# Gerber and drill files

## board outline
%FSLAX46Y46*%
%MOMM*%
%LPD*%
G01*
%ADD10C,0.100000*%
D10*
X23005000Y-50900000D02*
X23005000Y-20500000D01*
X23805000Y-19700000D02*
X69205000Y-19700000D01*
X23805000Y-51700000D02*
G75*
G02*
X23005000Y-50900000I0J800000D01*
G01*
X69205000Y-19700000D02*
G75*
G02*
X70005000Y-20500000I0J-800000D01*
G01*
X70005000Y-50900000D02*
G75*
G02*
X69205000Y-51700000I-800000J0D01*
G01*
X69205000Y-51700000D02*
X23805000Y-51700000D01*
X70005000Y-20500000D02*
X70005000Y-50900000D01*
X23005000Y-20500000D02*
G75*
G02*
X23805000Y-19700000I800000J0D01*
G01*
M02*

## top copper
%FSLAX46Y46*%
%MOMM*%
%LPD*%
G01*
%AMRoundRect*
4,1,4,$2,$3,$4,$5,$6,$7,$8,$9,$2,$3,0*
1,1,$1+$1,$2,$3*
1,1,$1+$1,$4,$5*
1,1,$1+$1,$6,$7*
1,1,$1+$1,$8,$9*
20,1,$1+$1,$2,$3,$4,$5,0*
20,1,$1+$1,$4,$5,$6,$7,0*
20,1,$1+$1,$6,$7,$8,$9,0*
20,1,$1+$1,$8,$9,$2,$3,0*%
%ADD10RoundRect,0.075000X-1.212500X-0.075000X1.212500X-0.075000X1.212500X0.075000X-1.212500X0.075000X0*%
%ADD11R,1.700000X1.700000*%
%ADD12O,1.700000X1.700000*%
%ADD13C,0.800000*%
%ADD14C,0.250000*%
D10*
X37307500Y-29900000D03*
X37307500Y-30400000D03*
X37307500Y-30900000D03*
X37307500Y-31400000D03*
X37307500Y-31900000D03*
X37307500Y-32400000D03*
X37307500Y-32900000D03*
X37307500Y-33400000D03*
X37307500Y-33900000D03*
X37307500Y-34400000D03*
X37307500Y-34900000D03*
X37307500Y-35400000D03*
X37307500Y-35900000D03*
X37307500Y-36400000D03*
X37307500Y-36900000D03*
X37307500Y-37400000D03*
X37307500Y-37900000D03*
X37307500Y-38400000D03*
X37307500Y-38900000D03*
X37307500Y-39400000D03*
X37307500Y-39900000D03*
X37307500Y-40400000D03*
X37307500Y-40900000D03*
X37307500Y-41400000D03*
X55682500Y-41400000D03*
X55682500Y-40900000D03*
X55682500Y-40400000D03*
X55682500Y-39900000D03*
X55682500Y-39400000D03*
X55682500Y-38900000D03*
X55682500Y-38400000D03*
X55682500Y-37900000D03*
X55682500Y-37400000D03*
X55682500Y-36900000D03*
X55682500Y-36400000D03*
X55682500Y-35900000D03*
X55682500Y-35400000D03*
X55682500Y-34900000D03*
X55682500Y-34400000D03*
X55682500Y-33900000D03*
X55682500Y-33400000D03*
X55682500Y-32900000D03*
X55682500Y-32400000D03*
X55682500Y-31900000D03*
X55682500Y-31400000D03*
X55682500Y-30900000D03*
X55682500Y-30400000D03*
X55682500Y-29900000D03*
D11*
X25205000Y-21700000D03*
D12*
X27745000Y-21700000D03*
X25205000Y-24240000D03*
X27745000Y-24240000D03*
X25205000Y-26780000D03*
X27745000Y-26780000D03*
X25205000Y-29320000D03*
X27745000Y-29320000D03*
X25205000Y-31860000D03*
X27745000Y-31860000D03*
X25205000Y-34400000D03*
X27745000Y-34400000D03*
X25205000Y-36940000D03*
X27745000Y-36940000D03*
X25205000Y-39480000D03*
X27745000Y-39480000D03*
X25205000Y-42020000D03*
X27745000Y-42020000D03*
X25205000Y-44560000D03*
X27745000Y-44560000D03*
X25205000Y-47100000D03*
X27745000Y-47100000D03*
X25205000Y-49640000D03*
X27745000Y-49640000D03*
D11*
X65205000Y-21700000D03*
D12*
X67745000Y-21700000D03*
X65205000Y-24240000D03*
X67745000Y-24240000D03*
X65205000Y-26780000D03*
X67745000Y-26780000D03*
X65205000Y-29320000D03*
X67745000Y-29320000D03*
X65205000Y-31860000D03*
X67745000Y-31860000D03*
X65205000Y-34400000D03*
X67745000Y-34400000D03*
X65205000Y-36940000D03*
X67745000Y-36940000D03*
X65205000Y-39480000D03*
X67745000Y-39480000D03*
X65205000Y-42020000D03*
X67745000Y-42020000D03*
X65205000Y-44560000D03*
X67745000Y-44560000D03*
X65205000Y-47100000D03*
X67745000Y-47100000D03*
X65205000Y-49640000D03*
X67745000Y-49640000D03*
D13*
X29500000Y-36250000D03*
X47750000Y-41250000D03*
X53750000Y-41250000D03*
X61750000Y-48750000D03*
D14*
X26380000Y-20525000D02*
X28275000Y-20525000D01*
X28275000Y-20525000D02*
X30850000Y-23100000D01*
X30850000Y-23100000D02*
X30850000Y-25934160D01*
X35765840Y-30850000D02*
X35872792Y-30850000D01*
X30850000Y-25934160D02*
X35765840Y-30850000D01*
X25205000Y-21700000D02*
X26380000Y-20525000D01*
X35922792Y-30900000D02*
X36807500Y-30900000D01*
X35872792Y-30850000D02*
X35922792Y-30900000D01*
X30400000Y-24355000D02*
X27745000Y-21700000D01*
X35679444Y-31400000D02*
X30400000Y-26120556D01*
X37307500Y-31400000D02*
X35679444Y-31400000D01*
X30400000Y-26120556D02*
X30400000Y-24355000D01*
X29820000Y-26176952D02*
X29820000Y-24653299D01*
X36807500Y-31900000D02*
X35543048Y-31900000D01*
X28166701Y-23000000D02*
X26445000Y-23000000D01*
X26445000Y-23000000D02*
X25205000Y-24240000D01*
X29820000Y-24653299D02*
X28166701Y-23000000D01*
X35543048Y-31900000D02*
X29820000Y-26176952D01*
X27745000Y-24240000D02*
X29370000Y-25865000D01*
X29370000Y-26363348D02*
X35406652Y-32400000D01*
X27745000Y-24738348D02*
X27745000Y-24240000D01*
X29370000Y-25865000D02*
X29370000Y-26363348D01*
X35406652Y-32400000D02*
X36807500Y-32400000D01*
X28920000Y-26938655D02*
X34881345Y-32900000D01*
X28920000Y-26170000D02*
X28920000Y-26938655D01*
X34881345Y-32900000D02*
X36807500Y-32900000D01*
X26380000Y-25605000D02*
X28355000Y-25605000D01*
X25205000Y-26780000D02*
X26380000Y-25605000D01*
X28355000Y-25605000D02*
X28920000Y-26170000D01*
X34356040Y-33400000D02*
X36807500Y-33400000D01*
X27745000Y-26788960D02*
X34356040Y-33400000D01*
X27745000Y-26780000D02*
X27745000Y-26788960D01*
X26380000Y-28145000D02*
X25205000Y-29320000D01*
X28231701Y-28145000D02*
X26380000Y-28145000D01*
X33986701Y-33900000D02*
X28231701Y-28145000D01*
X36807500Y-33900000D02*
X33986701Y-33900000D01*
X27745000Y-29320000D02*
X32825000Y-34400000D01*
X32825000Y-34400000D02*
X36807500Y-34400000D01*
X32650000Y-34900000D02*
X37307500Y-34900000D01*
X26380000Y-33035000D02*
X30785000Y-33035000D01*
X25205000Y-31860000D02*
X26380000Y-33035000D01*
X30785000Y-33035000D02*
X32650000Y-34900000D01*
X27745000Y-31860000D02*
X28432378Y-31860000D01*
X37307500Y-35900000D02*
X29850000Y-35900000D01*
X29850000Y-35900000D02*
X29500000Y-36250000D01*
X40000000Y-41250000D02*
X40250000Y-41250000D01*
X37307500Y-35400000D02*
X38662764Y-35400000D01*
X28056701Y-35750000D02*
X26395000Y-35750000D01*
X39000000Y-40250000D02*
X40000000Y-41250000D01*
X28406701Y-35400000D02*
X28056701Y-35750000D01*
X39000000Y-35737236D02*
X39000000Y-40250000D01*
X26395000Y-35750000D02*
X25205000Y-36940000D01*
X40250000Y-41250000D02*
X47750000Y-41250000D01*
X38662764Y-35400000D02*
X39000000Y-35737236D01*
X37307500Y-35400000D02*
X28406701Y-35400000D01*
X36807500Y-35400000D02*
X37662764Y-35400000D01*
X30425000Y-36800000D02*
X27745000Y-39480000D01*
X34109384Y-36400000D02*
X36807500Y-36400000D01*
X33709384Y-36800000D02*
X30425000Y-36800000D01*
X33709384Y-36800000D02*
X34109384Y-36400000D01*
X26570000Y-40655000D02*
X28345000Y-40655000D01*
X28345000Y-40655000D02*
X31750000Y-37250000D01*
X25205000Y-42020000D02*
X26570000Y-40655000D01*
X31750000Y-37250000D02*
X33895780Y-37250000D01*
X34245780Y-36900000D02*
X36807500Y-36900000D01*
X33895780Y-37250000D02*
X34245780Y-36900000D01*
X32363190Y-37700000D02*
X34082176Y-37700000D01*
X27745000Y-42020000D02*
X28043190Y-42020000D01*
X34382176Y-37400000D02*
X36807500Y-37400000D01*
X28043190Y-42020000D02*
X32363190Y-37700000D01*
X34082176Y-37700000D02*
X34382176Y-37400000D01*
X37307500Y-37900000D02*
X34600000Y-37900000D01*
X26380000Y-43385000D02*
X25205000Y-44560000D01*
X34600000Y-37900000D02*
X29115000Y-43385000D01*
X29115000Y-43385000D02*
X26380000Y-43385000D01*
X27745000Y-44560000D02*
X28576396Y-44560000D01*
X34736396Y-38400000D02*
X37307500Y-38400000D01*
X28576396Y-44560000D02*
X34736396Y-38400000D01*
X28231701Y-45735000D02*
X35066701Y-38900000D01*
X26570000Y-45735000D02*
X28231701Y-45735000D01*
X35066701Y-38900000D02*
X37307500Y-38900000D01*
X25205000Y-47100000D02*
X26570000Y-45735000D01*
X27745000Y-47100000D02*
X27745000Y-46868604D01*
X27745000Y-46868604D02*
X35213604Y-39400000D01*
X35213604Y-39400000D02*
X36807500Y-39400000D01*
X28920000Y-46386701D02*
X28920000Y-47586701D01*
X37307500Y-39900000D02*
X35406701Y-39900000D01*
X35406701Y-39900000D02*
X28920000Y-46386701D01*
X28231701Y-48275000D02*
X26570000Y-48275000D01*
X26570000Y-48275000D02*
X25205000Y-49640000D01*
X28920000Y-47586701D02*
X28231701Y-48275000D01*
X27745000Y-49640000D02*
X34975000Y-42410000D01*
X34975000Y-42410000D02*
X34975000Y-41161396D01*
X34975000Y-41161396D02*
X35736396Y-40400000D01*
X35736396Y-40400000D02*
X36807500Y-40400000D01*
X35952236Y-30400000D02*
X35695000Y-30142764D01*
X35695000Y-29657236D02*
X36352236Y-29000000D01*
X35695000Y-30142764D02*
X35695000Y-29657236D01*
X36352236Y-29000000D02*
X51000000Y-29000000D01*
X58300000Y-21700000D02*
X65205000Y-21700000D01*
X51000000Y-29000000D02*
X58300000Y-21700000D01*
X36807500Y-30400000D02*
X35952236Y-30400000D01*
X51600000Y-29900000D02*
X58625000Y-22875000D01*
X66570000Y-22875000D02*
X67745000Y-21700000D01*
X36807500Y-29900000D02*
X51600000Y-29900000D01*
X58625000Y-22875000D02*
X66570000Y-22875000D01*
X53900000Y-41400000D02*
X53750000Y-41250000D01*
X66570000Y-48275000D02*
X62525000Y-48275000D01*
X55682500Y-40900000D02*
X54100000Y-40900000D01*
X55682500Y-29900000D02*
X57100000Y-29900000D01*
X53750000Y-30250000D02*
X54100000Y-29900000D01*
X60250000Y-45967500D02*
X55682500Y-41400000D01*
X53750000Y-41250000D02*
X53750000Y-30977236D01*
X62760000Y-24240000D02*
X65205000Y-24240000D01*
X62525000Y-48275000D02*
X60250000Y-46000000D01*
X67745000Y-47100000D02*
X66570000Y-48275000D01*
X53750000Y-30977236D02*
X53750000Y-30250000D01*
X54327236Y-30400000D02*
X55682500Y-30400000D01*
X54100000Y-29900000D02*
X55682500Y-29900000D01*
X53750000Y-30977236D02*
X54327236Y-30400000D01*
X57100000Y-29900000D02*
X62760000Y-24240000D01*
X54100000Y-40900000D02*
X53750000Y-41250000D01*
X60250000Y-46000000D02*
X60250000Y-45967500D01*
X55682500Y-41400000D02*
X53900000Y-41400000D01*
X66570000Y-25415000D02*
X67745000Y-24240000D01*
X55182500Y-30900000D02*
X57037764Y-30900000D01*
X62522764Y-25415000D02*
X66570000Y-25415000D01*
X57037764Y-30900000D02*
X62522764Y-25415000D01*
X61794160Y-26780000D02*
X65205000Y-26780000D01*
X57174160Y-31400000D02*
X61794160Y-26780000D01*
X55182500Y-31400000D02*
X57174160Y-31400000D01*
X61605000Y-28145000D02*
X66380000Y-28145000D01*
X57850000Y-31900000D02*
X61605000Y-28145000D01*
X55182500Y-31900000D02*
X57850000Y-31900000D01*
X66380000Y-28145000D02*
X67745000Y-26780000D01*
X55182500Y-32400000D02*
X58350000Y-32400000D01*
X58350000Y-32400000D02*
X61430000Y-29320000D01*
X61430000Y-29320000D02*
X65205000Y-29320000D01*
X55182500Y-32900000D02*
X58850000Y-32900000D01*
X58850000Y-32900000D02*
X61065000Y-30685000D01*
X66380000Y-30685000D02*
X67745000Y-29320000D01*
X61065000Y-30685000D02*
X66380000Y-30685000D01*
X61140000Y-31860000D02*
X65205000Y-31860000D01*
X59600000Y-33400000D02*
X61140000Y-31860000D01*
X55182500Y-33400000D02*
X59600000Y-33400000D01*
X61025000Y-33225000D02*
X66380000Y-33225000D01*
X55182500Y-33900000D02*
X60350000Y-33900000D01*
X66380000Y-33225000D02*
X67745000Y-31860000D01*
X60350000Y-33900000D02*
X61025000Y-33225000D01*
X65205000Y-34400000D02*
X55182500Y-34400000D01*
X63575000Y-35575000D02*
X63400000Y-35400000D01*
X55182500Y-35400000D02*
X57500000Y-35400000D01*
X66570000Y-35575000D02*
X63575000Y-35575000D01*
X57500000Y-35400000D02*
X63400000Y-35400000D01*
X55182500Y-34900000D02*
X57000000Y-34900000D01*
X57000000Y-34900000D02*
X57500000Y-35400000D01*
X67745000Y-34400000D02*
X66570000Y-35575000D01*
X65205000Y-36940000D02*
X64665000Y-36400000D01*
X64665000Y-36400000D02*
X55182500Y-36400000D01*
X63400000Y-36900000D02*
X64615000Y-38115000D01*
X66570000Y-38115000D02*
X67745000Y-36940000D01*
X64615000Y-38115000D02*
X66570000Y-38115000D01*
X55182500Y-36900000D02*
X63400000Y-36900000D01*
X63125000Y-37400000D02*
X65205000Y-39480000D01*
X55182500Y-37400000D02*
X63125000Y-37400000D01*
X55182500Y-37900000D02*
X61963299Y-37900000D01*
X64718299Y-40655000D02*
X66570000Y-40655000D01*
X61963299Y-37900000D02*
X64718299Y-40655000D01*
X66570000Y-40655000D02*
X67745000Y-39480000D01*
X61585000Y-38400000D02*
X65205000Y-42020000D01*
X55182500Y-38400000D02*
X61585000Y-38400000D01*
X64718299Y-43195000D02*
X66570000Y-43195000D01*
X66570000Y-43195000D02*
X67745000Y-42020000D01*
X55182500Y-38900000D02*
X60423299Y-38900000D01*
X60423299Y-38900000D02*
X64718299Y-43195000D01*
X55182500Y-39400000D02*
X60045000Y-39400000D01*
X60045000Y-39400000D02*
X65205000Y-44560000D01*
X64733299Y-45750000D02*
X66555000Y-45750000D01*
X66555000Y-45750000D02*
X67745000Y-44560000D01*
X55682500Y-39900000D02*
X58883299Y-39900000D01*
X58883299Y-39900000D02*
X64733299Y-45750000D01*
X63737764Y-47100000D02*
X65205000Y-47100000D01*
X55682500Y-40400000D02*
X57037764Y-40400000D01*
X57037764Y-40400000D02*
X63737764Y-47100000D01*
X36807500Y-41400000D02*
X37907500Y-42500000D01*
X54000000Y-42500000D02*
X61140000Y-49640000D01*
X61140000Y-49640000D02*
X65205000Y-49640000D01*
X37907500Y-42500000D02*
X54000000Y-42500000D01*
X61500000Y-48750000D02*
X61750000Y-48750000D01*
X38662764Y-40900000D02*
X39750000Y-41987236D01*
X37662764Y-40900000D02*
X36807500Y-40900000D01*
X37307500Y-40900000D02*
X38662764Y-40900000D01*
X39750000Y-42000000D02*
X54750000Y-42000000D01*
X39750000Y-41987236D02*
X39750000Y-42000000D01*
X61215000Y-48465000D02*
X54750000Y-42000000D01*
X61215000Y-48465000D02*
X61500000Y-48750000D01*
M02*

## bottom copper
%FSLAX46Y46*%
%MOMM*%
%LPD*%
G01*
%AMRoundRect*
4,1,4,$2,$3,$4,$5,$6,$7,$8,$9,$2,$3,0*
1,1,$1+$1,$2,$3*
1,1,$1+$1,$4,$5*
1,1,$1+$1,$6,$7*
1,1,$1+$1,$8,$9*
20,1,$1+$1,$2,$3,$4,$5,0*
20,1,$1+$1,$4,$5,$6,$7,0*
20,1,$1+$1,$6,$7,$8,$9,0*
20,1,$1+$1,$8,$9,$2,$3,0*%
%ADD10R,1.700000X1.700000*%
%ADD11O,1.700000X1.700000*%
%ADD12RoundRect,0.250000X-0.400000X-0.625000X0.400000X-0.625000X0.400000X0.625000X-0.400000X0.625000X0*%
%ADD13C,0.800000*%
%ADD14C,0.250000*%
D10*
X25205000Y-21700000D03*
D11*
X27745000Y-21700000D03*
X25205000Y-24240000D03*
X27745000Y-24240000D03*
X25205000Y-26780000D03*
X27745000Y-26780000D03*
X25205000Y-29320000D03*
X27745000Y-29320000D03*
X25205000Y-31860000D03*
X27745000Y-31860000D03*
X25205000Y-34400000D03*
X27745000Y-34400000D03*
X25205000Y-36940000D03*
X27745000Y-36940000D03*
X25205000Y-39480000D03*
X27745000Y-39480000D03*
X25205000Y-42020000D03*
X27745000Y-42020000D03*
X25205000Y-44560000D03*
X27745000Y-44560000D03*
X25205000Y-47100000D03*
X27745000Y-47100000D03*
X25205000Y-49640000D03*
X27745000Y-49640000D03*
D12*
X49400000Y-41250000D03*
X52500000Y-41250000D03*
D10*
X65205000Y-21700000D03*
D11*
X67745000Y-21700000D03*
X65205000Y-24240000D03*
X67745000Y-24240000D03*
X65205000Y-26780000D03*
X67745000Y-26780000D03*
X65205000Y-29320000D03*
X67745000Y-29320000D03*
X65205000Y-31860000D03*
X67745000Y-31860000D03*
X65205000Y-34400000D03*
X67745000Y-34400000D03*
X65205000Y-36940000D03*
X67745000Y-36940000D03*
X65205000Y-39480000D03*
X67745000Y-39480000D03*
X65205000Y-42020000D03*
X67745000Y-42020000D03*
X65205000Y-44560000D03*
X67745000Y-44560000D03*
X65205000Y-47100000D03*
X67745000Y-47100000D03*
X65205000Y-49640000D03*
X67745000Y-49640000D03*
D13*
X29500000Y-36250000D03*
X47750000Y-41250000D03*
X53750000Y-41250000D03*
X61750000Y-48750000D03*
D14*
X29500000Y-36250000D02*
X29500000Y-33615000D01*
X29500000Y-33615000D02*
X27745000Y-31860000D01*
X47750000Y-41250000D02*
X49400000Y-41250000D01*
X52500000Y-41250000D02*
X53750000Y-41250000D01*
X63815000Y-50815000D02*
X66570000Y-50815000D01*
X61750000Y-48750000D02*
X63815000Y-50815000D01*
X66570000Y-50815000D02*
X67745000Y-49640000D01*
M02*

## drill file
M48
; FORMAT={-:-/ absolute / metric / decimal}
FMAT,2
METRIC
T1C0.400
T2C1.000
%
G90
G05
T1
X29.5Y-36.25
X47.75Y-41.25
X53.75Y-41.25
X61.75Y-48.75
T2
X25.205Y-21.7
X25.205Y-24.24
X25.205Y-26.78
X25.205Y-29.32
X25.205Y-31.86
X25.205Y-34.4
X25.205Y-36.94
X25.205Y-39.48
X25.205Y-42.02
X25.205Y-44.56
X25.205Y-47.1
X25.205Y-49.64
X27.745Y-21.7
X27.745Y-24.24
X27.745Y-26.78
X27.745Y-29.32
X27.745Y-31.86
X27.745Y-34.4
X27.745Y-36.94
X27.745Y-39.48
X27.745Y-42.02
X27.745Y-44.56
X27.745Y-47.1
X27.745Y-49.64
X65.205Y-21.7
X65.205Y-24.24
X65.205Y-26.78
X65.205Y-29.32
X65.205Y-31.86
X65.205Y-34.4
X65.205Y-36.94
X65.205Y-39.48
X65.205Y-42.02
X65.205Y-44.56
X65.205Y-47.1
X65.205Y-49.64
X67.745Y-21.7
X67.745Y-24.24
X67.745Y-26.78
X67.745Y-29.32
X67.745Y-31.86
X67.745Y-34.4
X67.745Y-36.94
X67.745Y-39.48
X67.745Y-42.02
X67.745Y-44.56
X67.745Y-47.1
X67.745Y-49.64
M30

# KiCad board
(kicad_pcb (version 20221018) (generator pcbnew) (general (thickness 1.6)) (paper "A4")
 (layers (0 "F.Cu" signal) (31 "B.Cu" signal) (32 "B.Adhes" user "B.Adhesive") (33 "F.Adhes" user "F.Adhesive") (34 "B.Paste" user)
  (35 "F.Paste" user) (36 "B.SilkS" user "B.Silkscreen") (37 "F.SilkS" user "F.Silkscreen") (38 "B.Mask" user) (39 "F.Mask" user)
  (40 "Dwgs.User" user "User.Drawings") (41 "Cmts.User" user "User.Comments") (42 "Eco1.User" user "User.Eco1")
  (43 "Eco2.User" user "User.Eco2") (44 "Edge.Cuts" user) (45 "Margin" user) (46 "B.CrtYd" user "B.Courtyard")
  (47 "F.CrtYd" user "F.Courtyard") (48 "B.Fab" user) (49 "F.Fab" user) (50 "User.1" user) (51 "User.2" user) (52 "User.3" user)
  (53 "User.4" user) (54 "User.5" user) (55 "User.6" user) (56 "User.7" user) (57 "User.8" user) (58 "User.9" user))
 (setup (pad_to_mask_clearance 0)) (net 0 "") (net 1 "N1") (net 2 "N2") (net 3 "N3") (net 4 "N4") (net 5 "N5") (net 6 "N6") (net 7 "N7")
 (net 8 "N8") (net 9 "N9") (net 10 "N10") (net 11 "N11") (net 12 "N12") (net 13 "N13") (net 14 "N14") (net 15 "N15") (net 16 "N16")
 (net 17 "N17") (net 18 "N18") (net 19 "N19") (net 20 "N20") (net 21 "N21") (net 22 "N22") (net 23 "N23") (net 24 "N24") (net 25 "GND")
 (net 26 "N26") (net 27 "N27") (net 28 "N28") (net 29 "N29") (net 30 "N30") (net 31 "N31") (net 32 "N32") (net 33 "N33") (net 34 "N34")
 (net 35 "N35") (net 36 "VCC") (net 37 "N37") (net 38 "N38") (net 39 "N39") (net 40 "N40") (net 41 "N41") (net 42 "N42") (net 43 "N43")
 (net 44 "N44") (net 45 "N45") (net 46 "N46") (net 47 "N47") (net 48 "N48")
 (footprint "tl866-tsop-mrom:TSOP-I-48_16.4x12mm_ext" (layer "F.Cu") (at 46.495 35.65)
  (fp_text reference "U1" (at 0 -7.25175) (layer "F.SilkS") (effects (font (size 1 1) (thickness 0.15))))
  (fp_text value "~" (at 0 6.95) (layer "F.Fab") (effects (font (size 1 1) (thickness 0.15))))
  (pad "1" smd roundrect (at -9.1875 -5.75) (size 2.575 0.3) (layers "F.Cu" "F.Paste" "F.Mask") (roundrect_rratio 0.25) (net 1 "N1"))
  (pad "2" smd roundrect (at -9.1875 -5.25) (size 2.575 0.3) (layers "F.Cu" "F.Paste" "F.Mask") (roundrect_rratio 0.25) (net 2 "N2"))
  (pad "3" smd roundrect (at -9.1875 -4.75) (size 2.575 0.3) (layers "F.Cu" "F.Paste" "F.Mask") (roundrect_rratio 0.25) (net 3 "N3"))
  (pad "4" smd roundrect (at -9.1875 -4.25) (size 2.575 0.3) (layers "F.Cu" "F.Paste" "F.Mask") (roundrect_rratio 0.25) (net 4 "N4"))
  (pad "5" smd roundrect (at -9.1875 -3.75) (size 2.575 0.3) (layers "F.Cu" "F.Paste" "F.Mask") (roundrect_rratio 0.25) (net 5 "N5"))
  (pad "6" smd roundrect (at -9.1875 -3.25) (size 2.575 0.3) (layers "F.Cu" "F.Paste" "F.Mask") (roundrect_rratio 0.25) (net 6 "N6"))
  (pad "7" smd roundrect (at -9.1875 -2.75) (size 2.575 0.3) (layers "F.Cu" "F.Paste" "F.Mask") (roundrect_rratio 0.25) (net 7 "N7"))
  (pad "8" smd roundrect (at -9.1875 -2.25) (size 2.575 0.3) (layers "F.Cu" "F.Paste" "F.Mask") (roundrect_rratio 0.25) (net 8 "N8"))
  (pad "9" smd roundrect (at -9.1875 -1.75) (size 2.575 0.3) (layers "F.Cu" "F.Paste" "F.Mask") (roundrect_rratio 0.25) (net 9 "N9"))
  (pad "10" smd roundrect (at -9.1875 -1.25) (size 2.575 0.3) (layers "F.Cu" "F.Paste" "F.Mask") (roundrect_rratio 0.25) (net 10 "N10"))
  (pad "11" smd roundrect (at -9.1875 -0.75) (size 2.575 0.3) (layers "F.Cu" "F.Paste" "F.Mask") (roundrect_rratio 0.25) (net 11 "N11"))
  (pad "12" smd roundrect (at -9.1875 -0.25) (size 2.575 0.3) (layers "F.Cu" "F.Paste" "F.Mask") (roundrect_rratio 0.25) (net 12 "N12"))
  (pad "13" smd roundrect (at -9.1875 0.25) (size 2.575 0.3) (layers "F.Cu" "F.Paste" "F.Mask") (roundrect_rratio 0.25) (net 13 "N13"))
  (pad "14" smd roundrect (at -9.1875 0.75) (size 2.575 0.3) (layers "F.Cu" "F.Paste" "F.Mask") (roundrect_rratio 0.25) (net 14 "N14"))
  (pad "15" smd roundrect (at -9.1875 1.25) (size 2.575 0.3) (layers "F.Cu" "F.Paste" "F.Mask") (roundrect_rratio 0.25) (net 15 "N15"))
  (pad "16" smd roundrect (at -9.1875 1.75) (size 2.575 0.3) (layers "F.Cu" "F.Paste" "F.Mask") (roundrect_rratio 0.25) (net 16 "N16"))
  (pad "17" smd roundrect (at -9.1875 2.25) (size 2.575 0.3) (layers "F.Cu" "F.Paste" "F.Mask") (roundrect_rratio 0.25) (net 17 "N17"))
  (pad "18" smd roundrect (at -9.1875 2.75) (size 2.575 0.3) (layers "F.Cu" "F.Paste" "F.Mask") (roundrect_rratio 0.25) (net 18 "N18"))
  (pad "19" smd roundrect (at -9.1875 3.25) (size 2.575 0.3) (layers "F.Cu" "F.Paste" "F.Mask") (roundrect_rratio 0.25) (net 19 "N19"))
  (pad "20" smd roundrect (at -9.1875 3.75) (size 2.575 0.3) (layers "F.Cu" "F.Paste" "F.Mask") (roundrect_rratio 0.25) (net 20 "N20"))
  (pad "21" smd roundrect (at -9.1875 4.25) (size 2.575 0.3) (layers "F.Cu" "F.Paste" "F.Mask") (roundrect_rratio 0.25) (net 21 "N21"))
  (pad "22" smd roundrect (at -9.1875 4.75) (size 2.575 0.3) (layers "F.Cu" "F.Paste" "F.Mask") (roundrect_rratio 0.25) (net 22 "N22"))
  (pad "23" smd roundrect (at -9.1875 5.25) (size 2.575 0.3) (layers "F.Cu" "F.Paste" "F.Mask") (roundrect_rratio 0.25) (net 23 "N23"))
  (pad "24" smd roundrect (at -9.1875 5.75) (size 2.575 0.3) (layers "F.Cu" "F.Paste" "F.Mask") (roundrect_rratio 0.25) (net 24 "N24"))
  (pad "25" smd roundrect (at 9.1875 5.75) (size 2.575 0.3) (layers "F.Cu" "F.Paste" "F.Mask") (roundrect_rratio 0.25) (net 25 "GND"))
  (pad "26" smd roundrect (at 9.1875 5.25) (size 2.575 0.3) (layers "F.Cu" "F.Paste" "F.Mask") (roundrect_rratio 0.25) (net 25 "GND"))
  (pad "27" smd roundrect (at 9.1875 4.75) (size 2.575 0.3) (layers "F.Cu" "F.Paste" "F.Mask") (roundrect_rratio 0.25) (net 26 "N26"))
  (pad "28" smd roundrect (at 9.1875 4.25) (size 2.575 0.3) (layers "F.Cu" "F.Paste" "F.Mask") (roundrect_rratio 0.25) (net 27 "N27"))
  (pad "29" smd roundrect (at 9.1875 3.75) (size 2.575 0.3) (layers "F.Cu" "F.Paste" "F.Mask") (roundrect_rratio 0.25) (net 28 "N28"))
  (pad "30" smd roundrect (at 9.1875 3.25) (size 2.575 0.3) (layers "F.Cu" "F.Paste" "F.Mask") (roundrect_rratio 0.25) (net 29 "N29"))
  (pad "31" smd roundrect (at 9.1875 2.75) (size 2.575 0.3) (layers "F.Cu" "F.Paste" "F.Mask") (roundrect_rratio 0.25) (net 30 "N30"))
  (pad "32" smd roundrect (at 9.1875 2.25) (size 2.575 0.3) (layers "F.Cu" "F.Paste" "F.Mask") (roundrect_rratio 0.25) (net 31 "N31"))
  (pad "33" smd roundrect (at 9.1875 1.75) (size 2.575 0.3) (layers "F.Cu" "F.Paste" "F.Mask") (roundrect_rratio 0.25) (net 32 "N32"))
  (pad "34" smd roundrect (at 9.1875 1.25) (size 2.575 0.3) (layers "F.Cu" "F.Paste" "F.Mask") (roundrect_rratio 0.25) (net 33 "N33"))
  (pad "35" smd roundrect (at 9.1875 0.75) (size 2.575 0.3) (layers "F.Cu" "F.Paste" "F.Mask") (roundrect_rratio 0.25) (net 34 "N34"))
  (pad "36" smd roundrect (at 9.1875 0.25) (size 2.575 0.3) (layers "F.Cu" "F.Paste" "F.Mask") (roundrect_rratio 0.25) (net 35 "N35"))
  (pad "37" smd roundrect (at 9.1875 -0.25) (size 2.575 0.3) (layers "F.Cu" "F.Paste" "F.Mask") (roundrect_rratio 0.25) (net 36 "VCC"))
  (pad "38" smd roundrect (at 9.1875 -0.75) (size 2.575 0.3) (layers "F.Cu" "F.Paste" "F.Mask") (roundrect_rratio 0.25) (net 36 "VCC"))
  (pad "39" smd roundrect (at 9.1875 -1.25) (size 2.575 0.3) (layers "F.Cu" "F.Paste" "F.Mask") (roundrect_rratio 0.25) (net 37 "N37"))
  (pad "40" smd roundrect (at 9.1875 -1.75) (size 2.575 0.3) (layers "F.Cu" "F.Paste" "F.Mask") (roundrect_rratio 0.25) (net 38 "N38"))
  (pad "41" smd roundrect (at 9.1875 -2.25) (size 2.575 0.3) (layers "F.Cu" "F.Paste" "F.Mask") (roundrect_rratio 0.25) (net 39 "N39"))
  (pad "42" smd roundrect (at 9.1875 -2.75) (size 2.575 0.3) (layers "F.Cu" "F.Paste" "F.Mask") (roundrect_rratio 0.25) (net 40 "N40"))
  (pad "43" smd roundrect (at 9.1875 -3.25) (size 2.575 0.3) (layers "F.Cu" "F.Paste" "F.Mask") (roundrect_rratio 0.25) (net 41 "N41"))
  (pad "44" smd roundrect (at 9.1875 -3.75) (size 2.575 0.3) (layers "F.Cu" "F.Paste" "F.Mask") (roundrect_rratio 0.25) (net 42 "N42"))
  (pad "45" smd roundrect (at 9.1875 -4.25) (size 2.575 0.3) (layers "F.Cu" "F.Paste" "F.Mask") (roundrect_rratio 0.25) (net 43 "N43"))
  (pad "46" smd roundrect (at 9.1875 -4.75) (size 2.575 0.3) (layers "F.Cu" "F.Paste" "F.Mask") (roundrect_rratio 0.25) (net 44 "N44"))
  (pad "47" smd roundrect (at 9.1875 -5.25) (size 2.575 0.3) (layers "F.Cu" "F.Paste" "F.Mask") (roundrect_rratio 0.25) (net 25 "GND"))
  (pad "48" smd roundrect (at 9.1875 -5.75) (size 2.575 0.3) (layers "F.Cu" "F.Paste" "F.Mask") (roundrect_rratio 0.25) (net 25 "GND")))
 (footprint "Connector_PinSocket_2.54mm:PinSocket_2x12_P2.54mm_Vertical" (layer "B.Cu") (at 25.205 21.7 180)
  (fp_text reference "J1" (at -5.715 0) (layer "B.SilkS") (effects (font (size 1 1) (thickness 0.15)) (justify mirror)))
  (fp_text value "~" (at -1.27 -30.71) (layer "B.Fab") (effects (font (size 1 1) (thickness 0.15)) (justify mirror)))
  (pad "1" thru_hole rect (at 0 0 180) (size 1.7 1.7) (drill 1) (layers "*.Cu" "*.Mask") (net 3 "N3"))
  (pad "2" thru_hole oval (at -2.54 0 180) (size 1.7 1.7) (drill 1) (layers "*.Cu" "*.Mask") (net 4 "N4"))
  (pad "3" thru_hole oval (at 0 -2.54 180) (size 1.7 1.7) (drill 1) (layers "*.Cu" "*.Mask") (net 5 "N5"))
  (pad "4" thru_hole oval (at -2.54 -2.54 180) (size 1.7 1.7) (drill 1) (layers "*.Cu" "*.Mask") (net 6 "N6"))
  (pad "5" thru_hole oval (at 0 -5.08 180) (size 1.7 1.7) (drill 1) (layers "*.Cu" "*.Mask") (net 7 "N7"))
  (pad "6" thru_hole oval (at -2.54 -5.08 180) (size 1.7 1.7) (drill 1) (layers "*.Cu" "*.Mask") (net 8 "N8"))
  (pad "7" thru_hole oval (at 0 -7.62 180) (size 1.7 1.7) (drill 1) (layers "*.Cu" "*.Mask") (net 9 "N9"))
  (pad "8" thru_hole oval (at -2.54 -7.62 180) (size 1.7 1.7) (drill 1) (layers "*.Cu" "*.Mask") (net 10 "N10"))
  (pad "9" thru_hole oval (at 0 -10.16 180) (size 1.7 1.7) (drill 1) (layers "*.Cu" "*.Mask") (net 11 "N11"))
  (pad "10" thru_hole oval (at -2.54 -10.16 180) (size 1.7 1.7) (drill 1) (layers "*.Cu" "*.Mask") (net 13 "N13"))
  (pad "11" thru_hole oval (at 0 -12.7 180) (size 1.7 1.7) (drill 1) (layers "*.Cu" "*.Mask") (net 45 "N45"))
  (pad "12" thru_hole oval (at -2.54 -12.7 180) (size 1.7 1.7) (drill 1) (layers "*.Cu" "*.Mask") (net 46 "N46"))
  (pad "13" thru_hole oval (at 0 -15.24 180) (size 1.7 1.7) (drill 1) (layers "*.Cu" "*.Mask") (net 12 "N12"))
  (pad "14" thru_hole oval (at -2.54 -15.24 180) (size 1.7 1.7) (drill 1) (layers "*.Cu" "*.Mask") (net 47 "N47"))
  (pad "15" thru_hole oval (at 0 -17.78 180) (size 1.7 1.7) (drill 1) (layers "*.Cu" "*.Mask") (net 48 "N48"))
  (pad "16" thru_hole oval (at -2.54 -17.78 180) (size 1.7 1.7) (drill 1) (layers "*.Cu" "*.Mask") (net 14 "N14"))
  (pad "17" thru_hole oval (at 0 -20.32 180) (size 1.7 1.7) (drill 1) (layers "*.Cu" "*.Mask") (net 15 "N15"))
  (pad "18" thru_hole oval (at -2.54 -20.32 180) (size 1.7 1.7) (drill 1) (layers "*.Cu" "*.Mask") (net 16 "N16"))
  (pad "19" thru_hole oval (at 0 -22.86 180) (size 1.7 1.7) (drill 1) (layers "*.Cu" "*.Mask") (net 17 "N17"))
  (pad "20" thru_hole oval (at -2.54 -22.86 180) (size 1.7 1.7) (drill 1) (layers "*.Cu" "*.Mask") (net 18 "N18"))
  (pad "21" thru_hole oval (at 0 -25.4 180) (size 1.7 1.7) (drill 1) (layers "*.Cu" "*.Mask") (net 19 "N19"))
  (pad "22" thru_hole oval (at -2.54 -25.4 180) (size 1.7 1.7) (drill 1) (layers "*.Cu" "*.Mask") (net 20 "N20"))
  (pad "23" thru_hole oval (at 0 -27.94 180) (size 1.7 1.7) (drill 1) (layers "*.Cu" "*.Mask") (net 21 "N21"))
  (pad "24" thru_hole oval (at -2.54 -27.94 180) (size 1.7 1.7) (drill 1) (layers "*.Cu" "*.Mask") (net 22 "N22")))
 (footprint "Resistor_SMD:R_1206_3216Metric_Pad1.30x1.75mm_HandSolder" (layer "B.Cu") (at 50.95 41.25)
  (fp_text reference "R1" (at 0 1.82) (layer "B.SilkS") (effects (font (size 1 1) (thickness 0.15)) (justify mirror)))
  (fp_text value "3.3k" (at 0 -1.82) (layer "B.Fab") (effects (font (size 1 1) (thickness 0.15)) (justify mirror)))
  (pad "1" smd roundrect (at -1.55 0) (size 1.3 1.75) (layers "B.Cu" "B.Paste" "B.Mask") (roundrect_rratio 0.192308) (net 12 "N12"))
  (pad "2" smd roundrect (at 1.55 0) (size 1.3 1.75) (layers "B.Cu" "B.Paste" "B.Mask") (roundrect_rratio 0.192308) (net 25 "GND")))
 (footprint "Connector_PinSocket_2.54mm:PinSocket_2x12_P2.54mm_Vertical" (layer "B.Cu") (at 65.205 21.7 180)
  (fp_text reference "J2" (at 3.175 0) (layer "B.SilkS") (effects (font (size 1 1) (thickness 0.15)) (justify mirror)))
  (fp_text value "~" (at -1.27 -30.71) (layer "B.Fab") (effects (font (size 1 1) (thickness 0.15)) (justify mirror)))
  (pad "1" thru_hole rect (at 0 0 180) (size 1.7 1.7) (drill 1) (layers "*.Cu" "*.Mask") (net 2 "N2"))
  (pad "2" thru_hole oval (at -2.54 0 180) (size 1.7 1.7) (drill 1) (layers "*.Cu" "*.Mask") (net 1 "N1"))
  (pad "3" thru_hole oval (at 0 -2.54 180) (size 1.7 1.7) (drill 1) (layers "*.Cu" "*.Mask") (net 25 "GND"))
  (pad "4" thru_hole oval (at -2.54 -2.54 180) (size 1.7 1.7) (drill 1) (layers "*.Cu" "*.Mask") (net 44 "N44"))
  (pad "5" thru_hole oval (at 0 -5.08 180) (size 1.7 1.7) (drill 1) (layers "*.Cu" "*.Mask") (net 43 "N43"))
  (pad "6" thru_hole oval (at -2.54 -5.08 180) (size 1.7 1.7) (drill 1) (layers "*.Cu" "*.Mask") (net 42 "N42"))
  (pad "7" thru_hole oval (at 0 -7.62 180) (size 1.7 1.7) (drill 1) (layers "*.Cu" "*.Mask") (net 41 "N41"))
  (pad "8" thru_hole oval (at -2.54 -7.62 180) (size 1.7 1.7) (drill 1) (layers "*.Cu" "*.Mask") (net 40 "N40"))
  (pad "9" thru_hole oval (at 0 -10.16 180) (size 1.7 1.7) (drill 1) (layers "*.Cu" "*.Mask") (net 39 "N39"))
  (pad "10" thru_hole oval (at -2.54 -10.16 180) (size 1.7 1.7) (drill 1) (layers "*.Cu" "*.Mask") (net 38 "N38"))
  (pad "11" thru_hole oval (at 0 -12.7 180) (size 1.7 1.7) (drill 1) (layers "*.Cu" "*.Mask") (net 37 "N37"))
  (pad "12" thru_hole oval (at -2.54 -12.7 180) (size 1.7 1.7) (drill 1) (layers "*.Cu" "*.Mask") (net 36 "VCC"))
  (pad "13" thru_hole oval (at 0 -15.24 180) (size 1.7 1.7) (drill 1) (layers "*.Cu" "*.Mask") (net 34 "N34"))
  (pad "14" thru_hole oval (at -2.54 -15.24 180) (size 1.7 1.7) (drill 1) (layers "*.Cu" "*.Mask") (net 33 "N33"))
  (pad "15" thru_hole oval (at 0 -17.78 180) (size 1.7 1.7) (drill 1) (layers "*.Cu" "*.Mask") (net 32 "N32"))
  (pad "16" thru_hole oval (at -2.54 -17.78 180) (size 1.7 1.7) (drill 1) (layers "*.Cu" "*.Mask") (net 31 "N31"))
  (pad "17" thru_hole oval (at 0 -20.32 180) (size 1.7 1.7) (drill 1) (layers "*.Cu" "*.Mask") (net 30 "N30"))
  (pad "18" thru_hole oval (at -2.54 -20.32 180) (size 1.7 1.7) (drill 1) (layers "*.Cu" "*.Mask") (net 29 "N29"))
  (pad "19" thru_hole oval (at 0 -22.86 180) (size 1.7 1.7) (drill 1) (layers "*.Cu" "*.Mask") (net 28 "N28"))
  (pad "20" thru_hole oval (at -2.54 -22.86 180) (size 1.7 1.7) (drill 1) (layers "*.Cu" "*.Mask") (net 27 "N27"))
  (pad "21" thru_hole oval (at 0 -25.4 180) (size 1.7 1.7) (drill 1) (layers "*.Cu" "*.Mask") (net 26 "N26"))
  (pad "22" thru_hole oval (at -2.54 -25.4 180) (size 1.7 1.7) (drill 1) (layers "*.Cu" "*.Mask") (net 25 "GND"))
  (pad "23" thru_hole oval (at 0 -27.94 180) (size 1.7 1.7) (drill 1) (layers "*.Cu" "*.Mask") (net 24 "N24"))
  (pad "24" thru_hole oval (at -2.54 -27.94 180) (size 1.7 1.7) (drill 1) (layers "*.Cu" "*.Mask") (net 23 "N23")))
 (gr_line (start 23.005 50.9) (end 23.005 20.5) (stroke (width 0.1) (type default)) (layer "Edge.Cuts"))
 (gr_line (start 23.805 19.7) (end 69.205 19.7) (stroke (width 0.1) (type default)) (layer "Edge.Cuts"))
 (gr_arc (start 23.805 51.7) (mid 23.239315 51.465685) (end 23.005 50.9) (stroke (width 0.1) (type default)) (layer "Edge.Cuts"))
 (gr_arc (start 69.205 19.7) (mid 69.770685 19.934315) (end 70.005 20.5) (stroke (width 0.1) (type default)) (layer "Edge.Cuts"))
 (gr_arc (start 70.005 50.9) (mid 69.770685 51.465685) (end 69.205 51.7) (stroke (width 0.1) (type default)) (layer "Edge.Cuts"))
 (gr_line (start 69.205 51.7) (end 23.805 51.7) (stroke (width 0.1) (type default)) (layer "Edge.Cuts"))
 (gr_line (start 70.005 20.5) (end 70.005 50.9) (stroke (width 0.1) (type default)) (layer "Edge.Cuts"))
 (gr_arc (start 23.005 20.5) (mid 23.239315 19.934315) (end 23.805 19.7) (stroke (width 0.1) (type default)) (layer "Edge.Cuts"))
 (segment (start 26.38 20.525) (end 28.275 20.525) (width 0.25) (layer "F.Cu") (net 3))
 (segment (start 28.275 20.525) (end 30.85 23.1) (width 0.25) (layer "F.Cu") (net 3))
 (segment (start 30.85 23.1) (end 30.85 25.93416) (width 0.25) (layer "F.Cu") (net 3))
 (segment (start 35.76584 30.85) (end 35.872792 30.85) (width 0.25) (layer "F.Cu") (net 3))
 (segment (start 30.85 25.93416) (end 35.76584 30.85) (width 0.25) (layer "F.Cu") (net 3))
 (segment (start 25.205 21.7) (end 26.38 20.525) (width 0.25) (layer "F.Cu") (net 3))
 (segment (start 35.922792 30.9) (end 36.8075 30.9) (width 0.25) (layer "F.Cu") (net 3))
 (segment (start 35.872792 30.85) (end 35.922792 30.9) (width 0.25) (layer "F.Cu") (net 3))
 (segment (start 30.4 24.355) (end 27.745 21.7) (width 0.25) (layer "F.Cu") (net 4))
 (segment (start 35.679444 31.4) (end 30.4 26.120556) (width 0.25) (layer "F.Cu") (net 4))
 (segment (start 37.3075 31.4) (end 35.679444 31.4) (width 0.25) (layer "F.Cu") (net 4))
 (segment (start 30.4 26.120556) (end 30.4 24.355) (width 0.25) (layer "F.Cu") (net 4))
 (segment (start 29.82 26.176952) (end 29.82 24.653299) (width 0.25) (layer "F.Cu") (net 5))
 (segment (start 36.8075 31.9) (end 35.543048 31.9) (width 0.25) (layer "F.Cu") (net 5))
 (segment (start 28.166701 23) (end 26.445 23) (width 0.25) (layer "F.Cu") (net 5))
 (segment (start 26.445 23) (end 25.205 24.24) (width 0.25) (layer "F.Cu") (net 5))
 (segment (start 29.82 24.653299) (end 28.166701 23) (width 0.25) (layer "F.Cu") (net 5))
 (segment (start 35.543048 31.9) (end 29.82 26.176952) (width 0.25) (layer "F.Cu") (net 5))
 (segment (start 27.745 24.24) (end 29.37 25.865) (width 0.25) (layer "F.Cu") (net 6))
 (segment (start 29.37 26.363348) (end 35.406652 32.4) (width 0.25) (layer "F.Cu") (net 6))
 (segment (start 27.745 24.738348) (end 27.745 24.24) (width 0.25) (layer "F.Cu") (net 6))
 (segment (start 29.37 25.865) (end 29.37 26.363348) (width 0.25) (layer "F.Cu") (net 6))
 (segment (start 35.406652 32.4) (end 36.8075 32.4) (width 0.25) (layer "F.Cu") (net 6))
 (segment (start 28.92 26.938655) (end 34.881345 32.9) (width 0.25) (layer "F.Cu") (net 7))
 (segment (start 28.92 26.17) (end 28.92 26.938655) (width 0.25) (layer "F.Cu") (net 7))
 (segment (start 34.881345 32.9) (end 36.8075 32.9) (width 0.25) (layer "F.Cu") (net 7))
 (segment (start 26.38 25.605) (end 28.355 25.605) (width 0.25) (layer "F.Cu") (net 7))
 (segment (start 25.205 26.78) (end 26.38 25.605) (width 0.25) (layer "F.Cu") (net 7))
 (segment (start 28.355 25.605) (end 28.92 26.17) (width 0.25) (layer "F.Cu") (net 7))
 (segment (start 34.35604 33.4) (end 36.8075 33.4) (width 0.25) (layer "F.Cu") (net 8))
 (segment (start 27.745 26.78896) (end 34.35604 33.4) (width 0.25) (layer "F.Cu") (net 8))
 (segment (start 27.745 26.78) (end 27.745 26.78896) (width 0.25) (layer "F.Cu") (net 8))
 (segment (start 26.38 28.145) (end 25.205 29.32) (width 0.25) (layer "F.Cu") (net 9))
 (segment (start 28.231701 28.145) (end 26.38 28.145) (width 0.25) (layer "F.Cu") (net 9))
 (segment (start 33.986701 33.9) (end 28.231701 28.145) (width 0.25) (layer "F.Cu") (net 9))
 (segment (start 36.8075 33.9) (end 33.986701 33.9) (width 0.25) (layer "F.Cu") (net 9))
 (segment (start 27.745 29.32) (end 32.825 34.4) (width 0.25) (layer "F.Cu") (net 10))
 (segment (start 32.825 34.4) (end 36.8075 34.4) (width 0.25) (layer "F.Cu") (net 10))
 (segment (start 32.65 34.9) (end 37.3075 34.9) (width 0.25) (layer "F.Cu") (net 11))
 (segment (start 26.38 33.035) (end 30.785 33.035) (width 0.25) (layer "F.Cu") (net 11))
 (segment (start 25.205 31.86) (end 26.38 33.035) (width 0.25) (layer "F.Cu") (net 11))
 (segment (start 30.785 33.035) (end 32.65 34.9) (width 0.25) (layer "F.Cu") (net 11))
 (segment (start 27.745 31.86) (end 28.432378 31.86) (width 0.25) (layer "F.Cu") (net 13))
 (segment (start 37.3075 35.9) (end 29.85 35.9) (width 0.25) (layer "F.Cu") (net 13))
 (segment (start 29.85 35.9) (end 29.5 36.25) (width 0.25) (layer "F.Cu") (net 13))
 (via (at 29.5 36.25) (size 0.8) (drill 0.4) (layers "F.Cu" "B.Cu") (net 13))
 (segment (start 29.5 36.25) (end 29.5 33.615) (width 0.25) (layer "B.Cu") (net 13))
 (segment (start 29.5 33.615) (end 27.745 31.86) (width 0.25) (layer "B.Cu") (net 13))
 (segment (start 40 41.25) (end 40.25 41.25) (width 0.25) (layer "F.Cu") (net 12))
 (segment (start 37.3075 35.4) (end 38.662764 35.4) (width 0.25) (layer "F.Cu") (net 12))
 (segment (start 28.056701 35.75) (end 26.395 35.75) (width 0.25) (layer "F.Cu") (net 12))
 (segment (start 39 40.25) (end 40 41.25) (width 0.25) (layer "F.Cu") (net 12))
 (segment (start 28.406701 35.4) (end 28.056701 35.75) (width 0.25) (layer "F.Cu") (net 12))
 (segment (start 39 35.737236) (end 39 40.25) (width 0.25) (layer "F.Cu") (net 12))
 (segment (start 26.395 35.75) (end 25.205 36.94) (width 0.25) (layer "F.Cu") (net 12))
 (segment (start 40.25 41.25) (end 47.75 41.25) (width 0.25) (layer "F.Cu") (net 12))
 (segment (start 38.662764 35.4) (end 39 35.737236) (width 0.25) (layer "F.Cu") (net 12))
 (segment (start 37.3075 35.4) (end 28.406701 35.4) (width 0.25) (layer "F.Cu") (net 12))
 (segment (start 36.8075 35.4) (end 37.662764 35.4) (width 0.25) (layer "F.Cu") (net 12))
 (via (at 47.75 41.25) (size 0.8) (drill 0.4) (layers "F.Cu" "B.Cu") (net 12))
 (segment (start 47.75 41.25) (end 49.4 41.25) (width 0.25) (layer "B.Cu") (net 12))
 (segment (start 30.425 36.8) (end 27.745 39.48) (width 0.25) (layer "F.Cu") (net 14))
 (segment (start 34.109384 36.4) (end 36.8075 36.4) (width 0.25) (layer "F.Cu") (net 14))
 (segment (start 33.709384 36.8) (end 30.425 36.8) (width 0.25) (layer "F.Cu") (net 14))
 (segment (start 33.709384 36.8) (end 34.109384 36.4) (width 0.25) (layer "F.Cu") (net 14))
 (segment (start 26.57 40.655) (end 28.345 40.655) (width 0.25) (layer "F.Cu") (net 15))
 (segment (start 28.345 40.655) (end 31.75 37.25) (width 0.25) (layer "F.Cu") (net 15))
 (segment (start 25.205 42.02) (end 26.57 40.655) (width 0.25) (layer "F.Cu") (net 15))
 (segment (start 31.75 37.25) (end 33.89578 37.25) (width 0.25) (layer "F.Cu") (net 15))
 (segment (start 34.24578 36.9) (end 36.8075 36.9) (width 0.25) (layer "F.Cu") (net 15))
 (segment (start 33.89578 37.25) (end 34.24578 36.9) (width 0.25) (layer "F.Cu") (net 15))
 (segment (start 32.36319 37.7) (end 34.082176 37.7) (width 0.25) (layer "F.Cu") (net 16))
 (segment (start 27.745 42.02) (end 28.04319 42.02) (width 0.25) (layer "F.Cu") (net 16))
 (segment (start 34.382176 37.4) (end 36.8075 37.4) (width 0.25) (layer "F.Cu") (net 16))
 (segment (start 28.04319 42.02) (end 32.36319 37.7) (width 0.25) (layer "F.Cu") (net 16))
 (segment (start 34.082176 37.7) (end 34.382176 37.4) (width 0.25) (layer "F.Cu") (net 16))
 (segment (start 37.3075 37.9) (end 34.6 37.9) (width 0.25) (layer "F.Cu") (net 17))
 (segment (start 26.38 43.385) (end 25.205 44.56) (width 0.25) (layer "F.Cu") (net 17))
 (segment (start 34.6 37.9) (end 29.115 43.385) (width 0.25) (layer "F.Cu") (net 17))
 (segment (start 29.115 43.385) (end 26.38 43.385) (width 0.25) (layer "F.Cu") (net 17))
 (segment (start 27.745 44.56) (end 28.576396 44.56) (width 0.25) (layer "F.Cu") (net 18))
 (segment (start 34.736396 38.4) (end 37.3075 38.4) (width 0.25) (layer "F.Cu") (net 18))
 (segment (start 28.576396 44.56) (end 34.736396 38.4) (width 0.25) (layer "F.Cu") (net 18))
 (segment (start 28.231701 45.735) (end 35.066701 38.9) (width 0.25) (layer "F.Cu") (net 19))
 (segment (start 26.57 45.735) (end 28.231701 45.735) (width 0.25) (layer "F.Cu") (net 19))
 (segment (start 35.066701 38.9) (end 37.3075 38.9) (width 0.25) (layer "F.Cu") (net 19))
 (segment (start 25.205 47.1) (end 26.57 45.735) (width 0.25) (layer "F.Cu") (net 19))
 (segment (start 27.745 47.1) (end 27.745 46.868604) (width 0.25) (layer "F.Cu") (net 20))
 (segment (start 27.745 46.868604) (end 35.213604 39.4) (width 0.25) (layer "F.Cu") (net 20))
 (segment (start 35.213604 39.4) (end 36.8075 39.4) (width 0.25) (layer "F.Cu") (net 20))
 (segment (start 28.92 46.386701) (end 28.92 47.586701) (width 0.25) (layer "F.Cu") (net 21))
 (segment (start 37.3075 39.9) (end 35.406701 39.9) (width 0.25) (layer "F.Cu") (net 21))
 (segment (start 35.406701 39.9) (end 28.92 46.386701) (width 0.25) (layer "F.Cu") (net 21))
 (segment (start 28.231701 48.275) (end 26.57 48.275) (width 0.25) (layer "F.Cu") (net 21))
 (segment (start 26.57 48.275) (end 25.205 49.64) (width 0.25) (layer "F.Cu") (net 21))
 (segment (start 28.92 47.586701) (end 28.231701 48.275) (width 0.25) (layer "F.Cu") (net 21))
 (segment (start 27.745 49.64) (end 34.975 42.41) (width 0.25) (layer "F.Cu") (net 22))
 (segment (start 34.975 42.41) (end 34.975 41.161396) (width 0.25) (layer "F.Cu") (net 22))
 (segment (start 34.975 41.161396) (end 35.736396 40.4) (width 0.25) (layer "F.Cu") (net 22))
 (segment (start 35.736396 40.4) (end 36.8075 40.4) (width 0.25) (layer "F.Cu") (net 22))
 (segment (start 35.952236 30.4) (end 35.695 30.142764) (width 0.25) (layer "F.Cu") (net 2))
 (segment (start 35.695 29.657236) (end 36.352236 29) (width 0.25) (layer "F.Cu") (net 2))
 (segment (start 35.695 30.142764) (end 35.695 29.657236) (width 0.25) (layer "F.Cu") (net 2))
 (segment (start 36.352236 29) (end 51 29) (width 0.25) (layer "F.Cu") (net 2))
 (segment (start 58.3 21.7) (end 65.205 21.7) (width 0.25) (layer "F.Cu") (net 2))
 (segment (start 51 29) (end 58.3 21.7) (width 0.25) (layer "F.Cu") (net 2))
 (segment (start 36.8075 30.4) (end 35.952236 30.4) (width 0.25) (layer "F.Cu") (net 2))
 (segment (start 51.6 29.9) (end 58.625 22.875) (width 0.25) (layer "F.Cu") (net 1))
 (segment (start 66.57 22.875) (end 67.745 21.7) (width 0.25) (layer "F.Cu") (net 1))
 (segment (start 36.8075 29.9) (end 51.6 29.9) (width 0.25) (layer "F.Cu") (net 1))
 (segment (start 58.625 22.875) (end 66.57 22.875) (width 0.25) (layer "F.Cu") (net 1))
 (segment (start 53.9 41.4) (end 53.75 41.25) (width 0.25) (layer "F.Cu") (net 25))
 (segment (start 66.57 48.275) (end 62.525 48.275) (width 0.25) (layer "F.Cu") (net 25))
 (segment (start 55.6825 40.9) (end 54.1 40.9) (width 0.25) (layer "F.Cu") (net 25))
 (segment (start 55.6825 29.9) (end 57.1 29.9) (width 0.25) (layer "F.Cu") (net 25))
 (segment (start 53.75 30.25) (end 54.1 29.9) (width 0.25) (layer "F.Cu") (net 25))
 (segment (start 60.25 45.9675) (end 55.6825 41.4) (width 0.25) (layer "F.Cu") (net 25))
 (segment (start 53.75 41.25) (end 53.75 30.977236) (width 0.25) (layer "F.Cu") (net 25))
 (segment (start 62.76 24.24) (end 65.205 24.24) (width 0.25) (layer "F.Cu") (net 25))
 (segment (start 62.525 48.275) (end 60.25 46) (width 0.25) (layer "F.Cu") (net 25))
 (segment (start 67.745 47.1) (end 66.57 48.275) (width 0.25) (layer "F.Cu") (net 25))
 (segment (start 53.75 30.977236) (end 53.75 30.25) (width 0.25) (layer "F.Cu") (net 25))
 (segment (start 54.327236 30.4) (end 55.6825 30.4) (width 0.25) (layer "F.Cu") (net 25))
 (segment (start 54.1 29.9) (end 55.6825 29.9) (width 0.25) (layer "F.Cu") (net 25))
 (segment (start 53.75 30.977236) (end 54.327236 30.4) (width 0.25) (layer "F.Cu") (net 25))
 (segment (start 57.1 29.9) (end 62.76 24.24) (width 0.25) (layer "F.Cu") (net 25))
 (segment (start 54.1 40.9) (end 53.75 41.25) (width 0.25) (layer "F.Cu") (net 25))
 (segment (start 60.25 46) (end 60.25 45.9675) (width 0.25) (layer "F.Cu") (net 25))
 (segment (start 55.6825 41.4) (end 53.9 41.4) (width 0.25) (layer "F.Cu") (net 25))
 (via (at 53.75 41.25) (size 0.8) (drill 0.4) (layers "F.Cu" "B.Cu") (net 25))
 (segment (start 52.5 41.25) (end 53.75 41.25) (width 0.25) (layer "B.Cu") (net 25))
 (segment (start 66.57 25.415) (end 67.745 24.24) (width 0.25) (layer "F.Cu") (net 44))
 (segment (start 55.1825 30.9) (end 57.037764 30.9) (width 0.25) (layer "F.Cu") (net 44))
 (segment (start 62.522764 25.415) (end 66.57 25.415) (width 0.25) (layer "F.Cu") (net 44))
 (segment (start 57.037764 30.9) (end 62.522764 25.415) (width 0.25) (layer "F.Cu") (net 44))
 (segment (start 61.79416 26.78) (end 65.205 26.78) (width 0.25) (layer "F.Cu") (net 43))
 (segment (start 57.17416 31.4) (end 61.79416 26.78) (width 0.25) (layer "F.Cu") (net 43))
 (segment (start 55.1825 31.4) (end 57.17416 31.4) (width 0.25) (layer "F.Cu") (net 43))
 (segment (start 61.605 28.145) (end 66.38 28.145) (width 0.25) (layer "F.Cu") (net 42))
 (segment (start 57.85 31.9) (end 61.605 28.145) (width 0.25) (layer "F.Cu") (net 42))
 (segment (start 55.1825 31.9) (end 57.85 31.9) (width 0.25) (layer "F.Cu") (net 42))
 (segment (start 66.38 28.145) (end 67.745 26.78) (width 0.25) (layer "F.Cu") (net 42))
 (segment (start 55.1825 32.4) (end 58.35 32.4) (width 0.25) (layer "F.Cu") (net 41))
 (segment (start 58.35 32.4) (end 61.43 29.32) (width 0.25) (layer "F.Cu") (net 41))
 (segment (start 61.43 29.32) (end 65.205 29.32) (width 0.25) (layer "F.Cu") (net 41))
 (segment (start 55.1825 32.9) (end 58.85 32.9) (width 0.25) (layer "F.Cu") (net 40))
 (segment (start 58.85 32.9) (end 61.065 30.685) (width 0.25) (layer "F.Cu") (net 40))
 (segment (start 66.38 30.685) (end 67.745 29.32) (width 0.25) (layer "F.Cu") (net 40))
 (segment (start 61.065 30.685) (end 66.38 30.685) (width 0.25) (layer "F.Cu") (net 40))
 (segment (start 61.14 31.86) (end 65.205 31.86) (width 0.25) (layer "F.Cu") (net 39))
 (segment (start 59.6 33.4) (end 61.14 31.86) (width 0.25) (layer "F.Cu") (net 39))
 (segment (start 55.1825 33.4) (end 59.6 33.4) (width 0.25) (layer "F.Cu") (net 39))
 (segment (start 61.025 33.225) (end 66.38 33.225) (width 0.25) (layer "F.Cu") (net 38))
 (segment (start 55.1825 33.9) (end 60.35 33.9) (width 0.25) (layer "F.Cu") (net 38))
 (segment (start 66.38 33.225) (end 67.745 31.86) (width 0.25) (layer "F.Cu") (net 38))
 (segment (start 60.35 33.9) (end 61.025 33.225) (width 0.25) (layer "F.Cu") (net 38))
 (segment (start 65.205 34.4) (end 55.1825 34.4) (width 0.25) (layer "F.Cu") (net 37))
 (segment (start 63.575 35.575) (end 63.4 35.4) (width 0.25) (layer "F.Cu") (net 36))
 (segment (start 55.1825 35.4) (end 57.5 35.4) (width 0.25) (layer "F.Cu") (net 36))
 (segment (start 66.57 35.575) (end 63.575 35.575) (width 0.25) (layer "F.Cu") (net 36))
 (segment (start 57.5 35.4) (end 63.4 35.4) (width 0.25) (layer "F.Cu") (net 36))
 (segment (start 55.1825 34.9) (end 57 34.9) (width 0.25) (layer "F.Cu") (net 36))
 (segment (start 57 34.9) (end 57.5 35.4) (width 0.25) (layer "F.Cu") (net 36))
 (segment (start 67.745 34.4) (end 66.57 35.575) (width 0.25) (layer "F.Cu") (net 36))
 (segment (start 65.205 36.94) (end 64.665 36.4) (width 0.25) (layer "F.Cu") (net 34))
 (segment (start 64.665 36.4) (end 55.1825 36.4) (width 0.25) (layer "F.Cu") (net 34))
 (segment (start 63.4 36.9) (end 64.615 38.115) (width 0.25) (layer "F.Cu") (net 33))
 (segment (start 66.57 38.115) (end 67.745 36.94) (width 0.25) (layer "F.Cu") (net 33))
 (segment (start 64.615 38.115) (end 66.57 38.115) (width 0.25) (layer "F.Cu") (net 33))
 (segment (start 55.1825 36.9) (end 63.4 36.9) (width 0.25) (layer "F.Cu") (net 33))
 (segment (start 63.125 37.4) (end 65.205 39.48) (width 0.25) (layer "F.Cu") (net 32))
 (segment (start 55.1825 37.4) (end 63.125 37.4) (width 0.25) (layer "F.Cu") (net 32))
 (segment (start 55.1825 37.9) (end 61.963299 37.9) (width 0.25) (layer "F.Cu") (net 31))
 (segment (start 64.718299 40.655) (end 66.57 40.655) (width 0.25) (layer "F.Cu") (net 31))
 (segment (start 61.963299 37.9) (end 64.718299 40.655) (width 0.25) (layer "F.Cu") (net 31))
 (segment (start 66.57 40.655) (end 67.745 39.48) (width 0.25) (layer "F.Cu") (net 31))
 (segment (start 61.585 38.4) (end 65.205 42.02) (width 0.25) (layer "F.Cu") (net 30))
 (segment (start 55.1825 38.4) (end 61.585 38.4) (width 0.25) (layer "F.Cu") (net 30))
 (segment (start 64.718299 43.195) (end 66.57 43.195) (width 0.25) (layer "F.Cu") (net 29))
 (segment (start 66.57 43.195) (end 67.745 42.02) (width 0.25) (layer "F.Cu") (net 29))
 (segment (start 55.1825 38.9) (end 60.423299 38.9) (width 0.25) (layer "F.Cu") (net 29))
 (segment (start 60.423299 38.9) (end 64.718299 43.195) (width 0.25) (layer "F.Cu") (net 29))
 (segment (start 55.1825 39.4) (end 60.045 39.4) (width 0.25) (layer "F.Cu") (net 28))
 (segment (start 60.045 39.4) (end 65.205 44.56) (width 0.25) (layer "F.Cu") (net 28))
 (segment (start 64.733299 45.75) (end 66.555 45.75) (width 0.25) (layer "F.Cu") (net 27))
 (segment (start 66.555 45.75) (end 67.745 44.56) (width 0.25) (layer "F.Cu") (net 27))
 (segment (start 55.6825 39.9) (end 58.883299 39.9) (width 0.25) (layer "F.Cu") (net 27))
 (segment (start 58.883299 39.9) (end 64.733299 45.75) (width 0.25) (layer "F.Cu") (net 27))
 (segment (start 63.737764 47.1) (end 65.205 47.1) (width 0.25) (layer "F.Cu") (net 26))
 (segment (start 55.6825 40.4) (end 57.037764 40.4) (width 0.25) (layer "F.Cu") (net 26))
 (segment (start 57.037764 40.4) (end 63.737764 47.1) (width 0.25) (layer "F.Cu") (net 26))
 (segment (start 36.8075 41.4) (end 37.9075 42.5) (width 0.25) (layer "F.Cu") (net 24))
 (segment (start 54 42.5) (end 61.14 49.64) (width 0.25) (layer "F.Cu") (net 24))
 (segment (start 61.14 49.64) (end 65.205 49.64) (width 0.25) (layer "F.Cu") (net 24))
 (segment (start 37.9075 42.5) (end 54 42.5) (width 0.25) (layer "F.Cu") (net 24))
 (segment (start 61.5 48.75) (end 61.75 48.75) (width 0.25) (layer "F.Cu") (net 23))
 (segment (start 38.662764 40.9) (end 39.75 41.987236) (width 0.25) (layer "F.Cu") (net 23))
 (segment (start 37.662764 40.9) (end 36.8075 40.9) (width 0.25) (layer "F.Cu") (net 23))
 (segment (start 37.3075 40.9) (end 38.662764 40.9) (width 0.25) (layer "F.Cu") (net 23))
 (segment (start 39.75 42) (end 54.75 42) (width 0.25) (layer "F.Cu") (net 23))
 (segment (start 39.75 41.987236) (end 39.75 42) (width 0.25) (layer "F.Cu") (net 23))
 (segment (start 61.215 48.465) (end 54.75 42) (width 0.25) (layer "F.Cu") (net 23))
 (segment (start 61.215 48.465) (end 61.5 48.75) (width 0.25) (layer "F.Cu") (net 23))
 (via (at 61.75 48.75) (size 0.8) (drill 0.4) (layers "F.Cu" "B.Cu") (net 23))
 (segment (start 63.815 50.815) (end 66.57 50.815) (width 0.25) (layer "B.Cu") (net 23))
 (segment (start 61.75 48.75) (end 63.815 50.815) (width 0.25) (layer "B.Cu") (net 23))
 (segment (start 66.57 50.815) (end 67.745 49.64) (width 0.25) (layer "B.Cu") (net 23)))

